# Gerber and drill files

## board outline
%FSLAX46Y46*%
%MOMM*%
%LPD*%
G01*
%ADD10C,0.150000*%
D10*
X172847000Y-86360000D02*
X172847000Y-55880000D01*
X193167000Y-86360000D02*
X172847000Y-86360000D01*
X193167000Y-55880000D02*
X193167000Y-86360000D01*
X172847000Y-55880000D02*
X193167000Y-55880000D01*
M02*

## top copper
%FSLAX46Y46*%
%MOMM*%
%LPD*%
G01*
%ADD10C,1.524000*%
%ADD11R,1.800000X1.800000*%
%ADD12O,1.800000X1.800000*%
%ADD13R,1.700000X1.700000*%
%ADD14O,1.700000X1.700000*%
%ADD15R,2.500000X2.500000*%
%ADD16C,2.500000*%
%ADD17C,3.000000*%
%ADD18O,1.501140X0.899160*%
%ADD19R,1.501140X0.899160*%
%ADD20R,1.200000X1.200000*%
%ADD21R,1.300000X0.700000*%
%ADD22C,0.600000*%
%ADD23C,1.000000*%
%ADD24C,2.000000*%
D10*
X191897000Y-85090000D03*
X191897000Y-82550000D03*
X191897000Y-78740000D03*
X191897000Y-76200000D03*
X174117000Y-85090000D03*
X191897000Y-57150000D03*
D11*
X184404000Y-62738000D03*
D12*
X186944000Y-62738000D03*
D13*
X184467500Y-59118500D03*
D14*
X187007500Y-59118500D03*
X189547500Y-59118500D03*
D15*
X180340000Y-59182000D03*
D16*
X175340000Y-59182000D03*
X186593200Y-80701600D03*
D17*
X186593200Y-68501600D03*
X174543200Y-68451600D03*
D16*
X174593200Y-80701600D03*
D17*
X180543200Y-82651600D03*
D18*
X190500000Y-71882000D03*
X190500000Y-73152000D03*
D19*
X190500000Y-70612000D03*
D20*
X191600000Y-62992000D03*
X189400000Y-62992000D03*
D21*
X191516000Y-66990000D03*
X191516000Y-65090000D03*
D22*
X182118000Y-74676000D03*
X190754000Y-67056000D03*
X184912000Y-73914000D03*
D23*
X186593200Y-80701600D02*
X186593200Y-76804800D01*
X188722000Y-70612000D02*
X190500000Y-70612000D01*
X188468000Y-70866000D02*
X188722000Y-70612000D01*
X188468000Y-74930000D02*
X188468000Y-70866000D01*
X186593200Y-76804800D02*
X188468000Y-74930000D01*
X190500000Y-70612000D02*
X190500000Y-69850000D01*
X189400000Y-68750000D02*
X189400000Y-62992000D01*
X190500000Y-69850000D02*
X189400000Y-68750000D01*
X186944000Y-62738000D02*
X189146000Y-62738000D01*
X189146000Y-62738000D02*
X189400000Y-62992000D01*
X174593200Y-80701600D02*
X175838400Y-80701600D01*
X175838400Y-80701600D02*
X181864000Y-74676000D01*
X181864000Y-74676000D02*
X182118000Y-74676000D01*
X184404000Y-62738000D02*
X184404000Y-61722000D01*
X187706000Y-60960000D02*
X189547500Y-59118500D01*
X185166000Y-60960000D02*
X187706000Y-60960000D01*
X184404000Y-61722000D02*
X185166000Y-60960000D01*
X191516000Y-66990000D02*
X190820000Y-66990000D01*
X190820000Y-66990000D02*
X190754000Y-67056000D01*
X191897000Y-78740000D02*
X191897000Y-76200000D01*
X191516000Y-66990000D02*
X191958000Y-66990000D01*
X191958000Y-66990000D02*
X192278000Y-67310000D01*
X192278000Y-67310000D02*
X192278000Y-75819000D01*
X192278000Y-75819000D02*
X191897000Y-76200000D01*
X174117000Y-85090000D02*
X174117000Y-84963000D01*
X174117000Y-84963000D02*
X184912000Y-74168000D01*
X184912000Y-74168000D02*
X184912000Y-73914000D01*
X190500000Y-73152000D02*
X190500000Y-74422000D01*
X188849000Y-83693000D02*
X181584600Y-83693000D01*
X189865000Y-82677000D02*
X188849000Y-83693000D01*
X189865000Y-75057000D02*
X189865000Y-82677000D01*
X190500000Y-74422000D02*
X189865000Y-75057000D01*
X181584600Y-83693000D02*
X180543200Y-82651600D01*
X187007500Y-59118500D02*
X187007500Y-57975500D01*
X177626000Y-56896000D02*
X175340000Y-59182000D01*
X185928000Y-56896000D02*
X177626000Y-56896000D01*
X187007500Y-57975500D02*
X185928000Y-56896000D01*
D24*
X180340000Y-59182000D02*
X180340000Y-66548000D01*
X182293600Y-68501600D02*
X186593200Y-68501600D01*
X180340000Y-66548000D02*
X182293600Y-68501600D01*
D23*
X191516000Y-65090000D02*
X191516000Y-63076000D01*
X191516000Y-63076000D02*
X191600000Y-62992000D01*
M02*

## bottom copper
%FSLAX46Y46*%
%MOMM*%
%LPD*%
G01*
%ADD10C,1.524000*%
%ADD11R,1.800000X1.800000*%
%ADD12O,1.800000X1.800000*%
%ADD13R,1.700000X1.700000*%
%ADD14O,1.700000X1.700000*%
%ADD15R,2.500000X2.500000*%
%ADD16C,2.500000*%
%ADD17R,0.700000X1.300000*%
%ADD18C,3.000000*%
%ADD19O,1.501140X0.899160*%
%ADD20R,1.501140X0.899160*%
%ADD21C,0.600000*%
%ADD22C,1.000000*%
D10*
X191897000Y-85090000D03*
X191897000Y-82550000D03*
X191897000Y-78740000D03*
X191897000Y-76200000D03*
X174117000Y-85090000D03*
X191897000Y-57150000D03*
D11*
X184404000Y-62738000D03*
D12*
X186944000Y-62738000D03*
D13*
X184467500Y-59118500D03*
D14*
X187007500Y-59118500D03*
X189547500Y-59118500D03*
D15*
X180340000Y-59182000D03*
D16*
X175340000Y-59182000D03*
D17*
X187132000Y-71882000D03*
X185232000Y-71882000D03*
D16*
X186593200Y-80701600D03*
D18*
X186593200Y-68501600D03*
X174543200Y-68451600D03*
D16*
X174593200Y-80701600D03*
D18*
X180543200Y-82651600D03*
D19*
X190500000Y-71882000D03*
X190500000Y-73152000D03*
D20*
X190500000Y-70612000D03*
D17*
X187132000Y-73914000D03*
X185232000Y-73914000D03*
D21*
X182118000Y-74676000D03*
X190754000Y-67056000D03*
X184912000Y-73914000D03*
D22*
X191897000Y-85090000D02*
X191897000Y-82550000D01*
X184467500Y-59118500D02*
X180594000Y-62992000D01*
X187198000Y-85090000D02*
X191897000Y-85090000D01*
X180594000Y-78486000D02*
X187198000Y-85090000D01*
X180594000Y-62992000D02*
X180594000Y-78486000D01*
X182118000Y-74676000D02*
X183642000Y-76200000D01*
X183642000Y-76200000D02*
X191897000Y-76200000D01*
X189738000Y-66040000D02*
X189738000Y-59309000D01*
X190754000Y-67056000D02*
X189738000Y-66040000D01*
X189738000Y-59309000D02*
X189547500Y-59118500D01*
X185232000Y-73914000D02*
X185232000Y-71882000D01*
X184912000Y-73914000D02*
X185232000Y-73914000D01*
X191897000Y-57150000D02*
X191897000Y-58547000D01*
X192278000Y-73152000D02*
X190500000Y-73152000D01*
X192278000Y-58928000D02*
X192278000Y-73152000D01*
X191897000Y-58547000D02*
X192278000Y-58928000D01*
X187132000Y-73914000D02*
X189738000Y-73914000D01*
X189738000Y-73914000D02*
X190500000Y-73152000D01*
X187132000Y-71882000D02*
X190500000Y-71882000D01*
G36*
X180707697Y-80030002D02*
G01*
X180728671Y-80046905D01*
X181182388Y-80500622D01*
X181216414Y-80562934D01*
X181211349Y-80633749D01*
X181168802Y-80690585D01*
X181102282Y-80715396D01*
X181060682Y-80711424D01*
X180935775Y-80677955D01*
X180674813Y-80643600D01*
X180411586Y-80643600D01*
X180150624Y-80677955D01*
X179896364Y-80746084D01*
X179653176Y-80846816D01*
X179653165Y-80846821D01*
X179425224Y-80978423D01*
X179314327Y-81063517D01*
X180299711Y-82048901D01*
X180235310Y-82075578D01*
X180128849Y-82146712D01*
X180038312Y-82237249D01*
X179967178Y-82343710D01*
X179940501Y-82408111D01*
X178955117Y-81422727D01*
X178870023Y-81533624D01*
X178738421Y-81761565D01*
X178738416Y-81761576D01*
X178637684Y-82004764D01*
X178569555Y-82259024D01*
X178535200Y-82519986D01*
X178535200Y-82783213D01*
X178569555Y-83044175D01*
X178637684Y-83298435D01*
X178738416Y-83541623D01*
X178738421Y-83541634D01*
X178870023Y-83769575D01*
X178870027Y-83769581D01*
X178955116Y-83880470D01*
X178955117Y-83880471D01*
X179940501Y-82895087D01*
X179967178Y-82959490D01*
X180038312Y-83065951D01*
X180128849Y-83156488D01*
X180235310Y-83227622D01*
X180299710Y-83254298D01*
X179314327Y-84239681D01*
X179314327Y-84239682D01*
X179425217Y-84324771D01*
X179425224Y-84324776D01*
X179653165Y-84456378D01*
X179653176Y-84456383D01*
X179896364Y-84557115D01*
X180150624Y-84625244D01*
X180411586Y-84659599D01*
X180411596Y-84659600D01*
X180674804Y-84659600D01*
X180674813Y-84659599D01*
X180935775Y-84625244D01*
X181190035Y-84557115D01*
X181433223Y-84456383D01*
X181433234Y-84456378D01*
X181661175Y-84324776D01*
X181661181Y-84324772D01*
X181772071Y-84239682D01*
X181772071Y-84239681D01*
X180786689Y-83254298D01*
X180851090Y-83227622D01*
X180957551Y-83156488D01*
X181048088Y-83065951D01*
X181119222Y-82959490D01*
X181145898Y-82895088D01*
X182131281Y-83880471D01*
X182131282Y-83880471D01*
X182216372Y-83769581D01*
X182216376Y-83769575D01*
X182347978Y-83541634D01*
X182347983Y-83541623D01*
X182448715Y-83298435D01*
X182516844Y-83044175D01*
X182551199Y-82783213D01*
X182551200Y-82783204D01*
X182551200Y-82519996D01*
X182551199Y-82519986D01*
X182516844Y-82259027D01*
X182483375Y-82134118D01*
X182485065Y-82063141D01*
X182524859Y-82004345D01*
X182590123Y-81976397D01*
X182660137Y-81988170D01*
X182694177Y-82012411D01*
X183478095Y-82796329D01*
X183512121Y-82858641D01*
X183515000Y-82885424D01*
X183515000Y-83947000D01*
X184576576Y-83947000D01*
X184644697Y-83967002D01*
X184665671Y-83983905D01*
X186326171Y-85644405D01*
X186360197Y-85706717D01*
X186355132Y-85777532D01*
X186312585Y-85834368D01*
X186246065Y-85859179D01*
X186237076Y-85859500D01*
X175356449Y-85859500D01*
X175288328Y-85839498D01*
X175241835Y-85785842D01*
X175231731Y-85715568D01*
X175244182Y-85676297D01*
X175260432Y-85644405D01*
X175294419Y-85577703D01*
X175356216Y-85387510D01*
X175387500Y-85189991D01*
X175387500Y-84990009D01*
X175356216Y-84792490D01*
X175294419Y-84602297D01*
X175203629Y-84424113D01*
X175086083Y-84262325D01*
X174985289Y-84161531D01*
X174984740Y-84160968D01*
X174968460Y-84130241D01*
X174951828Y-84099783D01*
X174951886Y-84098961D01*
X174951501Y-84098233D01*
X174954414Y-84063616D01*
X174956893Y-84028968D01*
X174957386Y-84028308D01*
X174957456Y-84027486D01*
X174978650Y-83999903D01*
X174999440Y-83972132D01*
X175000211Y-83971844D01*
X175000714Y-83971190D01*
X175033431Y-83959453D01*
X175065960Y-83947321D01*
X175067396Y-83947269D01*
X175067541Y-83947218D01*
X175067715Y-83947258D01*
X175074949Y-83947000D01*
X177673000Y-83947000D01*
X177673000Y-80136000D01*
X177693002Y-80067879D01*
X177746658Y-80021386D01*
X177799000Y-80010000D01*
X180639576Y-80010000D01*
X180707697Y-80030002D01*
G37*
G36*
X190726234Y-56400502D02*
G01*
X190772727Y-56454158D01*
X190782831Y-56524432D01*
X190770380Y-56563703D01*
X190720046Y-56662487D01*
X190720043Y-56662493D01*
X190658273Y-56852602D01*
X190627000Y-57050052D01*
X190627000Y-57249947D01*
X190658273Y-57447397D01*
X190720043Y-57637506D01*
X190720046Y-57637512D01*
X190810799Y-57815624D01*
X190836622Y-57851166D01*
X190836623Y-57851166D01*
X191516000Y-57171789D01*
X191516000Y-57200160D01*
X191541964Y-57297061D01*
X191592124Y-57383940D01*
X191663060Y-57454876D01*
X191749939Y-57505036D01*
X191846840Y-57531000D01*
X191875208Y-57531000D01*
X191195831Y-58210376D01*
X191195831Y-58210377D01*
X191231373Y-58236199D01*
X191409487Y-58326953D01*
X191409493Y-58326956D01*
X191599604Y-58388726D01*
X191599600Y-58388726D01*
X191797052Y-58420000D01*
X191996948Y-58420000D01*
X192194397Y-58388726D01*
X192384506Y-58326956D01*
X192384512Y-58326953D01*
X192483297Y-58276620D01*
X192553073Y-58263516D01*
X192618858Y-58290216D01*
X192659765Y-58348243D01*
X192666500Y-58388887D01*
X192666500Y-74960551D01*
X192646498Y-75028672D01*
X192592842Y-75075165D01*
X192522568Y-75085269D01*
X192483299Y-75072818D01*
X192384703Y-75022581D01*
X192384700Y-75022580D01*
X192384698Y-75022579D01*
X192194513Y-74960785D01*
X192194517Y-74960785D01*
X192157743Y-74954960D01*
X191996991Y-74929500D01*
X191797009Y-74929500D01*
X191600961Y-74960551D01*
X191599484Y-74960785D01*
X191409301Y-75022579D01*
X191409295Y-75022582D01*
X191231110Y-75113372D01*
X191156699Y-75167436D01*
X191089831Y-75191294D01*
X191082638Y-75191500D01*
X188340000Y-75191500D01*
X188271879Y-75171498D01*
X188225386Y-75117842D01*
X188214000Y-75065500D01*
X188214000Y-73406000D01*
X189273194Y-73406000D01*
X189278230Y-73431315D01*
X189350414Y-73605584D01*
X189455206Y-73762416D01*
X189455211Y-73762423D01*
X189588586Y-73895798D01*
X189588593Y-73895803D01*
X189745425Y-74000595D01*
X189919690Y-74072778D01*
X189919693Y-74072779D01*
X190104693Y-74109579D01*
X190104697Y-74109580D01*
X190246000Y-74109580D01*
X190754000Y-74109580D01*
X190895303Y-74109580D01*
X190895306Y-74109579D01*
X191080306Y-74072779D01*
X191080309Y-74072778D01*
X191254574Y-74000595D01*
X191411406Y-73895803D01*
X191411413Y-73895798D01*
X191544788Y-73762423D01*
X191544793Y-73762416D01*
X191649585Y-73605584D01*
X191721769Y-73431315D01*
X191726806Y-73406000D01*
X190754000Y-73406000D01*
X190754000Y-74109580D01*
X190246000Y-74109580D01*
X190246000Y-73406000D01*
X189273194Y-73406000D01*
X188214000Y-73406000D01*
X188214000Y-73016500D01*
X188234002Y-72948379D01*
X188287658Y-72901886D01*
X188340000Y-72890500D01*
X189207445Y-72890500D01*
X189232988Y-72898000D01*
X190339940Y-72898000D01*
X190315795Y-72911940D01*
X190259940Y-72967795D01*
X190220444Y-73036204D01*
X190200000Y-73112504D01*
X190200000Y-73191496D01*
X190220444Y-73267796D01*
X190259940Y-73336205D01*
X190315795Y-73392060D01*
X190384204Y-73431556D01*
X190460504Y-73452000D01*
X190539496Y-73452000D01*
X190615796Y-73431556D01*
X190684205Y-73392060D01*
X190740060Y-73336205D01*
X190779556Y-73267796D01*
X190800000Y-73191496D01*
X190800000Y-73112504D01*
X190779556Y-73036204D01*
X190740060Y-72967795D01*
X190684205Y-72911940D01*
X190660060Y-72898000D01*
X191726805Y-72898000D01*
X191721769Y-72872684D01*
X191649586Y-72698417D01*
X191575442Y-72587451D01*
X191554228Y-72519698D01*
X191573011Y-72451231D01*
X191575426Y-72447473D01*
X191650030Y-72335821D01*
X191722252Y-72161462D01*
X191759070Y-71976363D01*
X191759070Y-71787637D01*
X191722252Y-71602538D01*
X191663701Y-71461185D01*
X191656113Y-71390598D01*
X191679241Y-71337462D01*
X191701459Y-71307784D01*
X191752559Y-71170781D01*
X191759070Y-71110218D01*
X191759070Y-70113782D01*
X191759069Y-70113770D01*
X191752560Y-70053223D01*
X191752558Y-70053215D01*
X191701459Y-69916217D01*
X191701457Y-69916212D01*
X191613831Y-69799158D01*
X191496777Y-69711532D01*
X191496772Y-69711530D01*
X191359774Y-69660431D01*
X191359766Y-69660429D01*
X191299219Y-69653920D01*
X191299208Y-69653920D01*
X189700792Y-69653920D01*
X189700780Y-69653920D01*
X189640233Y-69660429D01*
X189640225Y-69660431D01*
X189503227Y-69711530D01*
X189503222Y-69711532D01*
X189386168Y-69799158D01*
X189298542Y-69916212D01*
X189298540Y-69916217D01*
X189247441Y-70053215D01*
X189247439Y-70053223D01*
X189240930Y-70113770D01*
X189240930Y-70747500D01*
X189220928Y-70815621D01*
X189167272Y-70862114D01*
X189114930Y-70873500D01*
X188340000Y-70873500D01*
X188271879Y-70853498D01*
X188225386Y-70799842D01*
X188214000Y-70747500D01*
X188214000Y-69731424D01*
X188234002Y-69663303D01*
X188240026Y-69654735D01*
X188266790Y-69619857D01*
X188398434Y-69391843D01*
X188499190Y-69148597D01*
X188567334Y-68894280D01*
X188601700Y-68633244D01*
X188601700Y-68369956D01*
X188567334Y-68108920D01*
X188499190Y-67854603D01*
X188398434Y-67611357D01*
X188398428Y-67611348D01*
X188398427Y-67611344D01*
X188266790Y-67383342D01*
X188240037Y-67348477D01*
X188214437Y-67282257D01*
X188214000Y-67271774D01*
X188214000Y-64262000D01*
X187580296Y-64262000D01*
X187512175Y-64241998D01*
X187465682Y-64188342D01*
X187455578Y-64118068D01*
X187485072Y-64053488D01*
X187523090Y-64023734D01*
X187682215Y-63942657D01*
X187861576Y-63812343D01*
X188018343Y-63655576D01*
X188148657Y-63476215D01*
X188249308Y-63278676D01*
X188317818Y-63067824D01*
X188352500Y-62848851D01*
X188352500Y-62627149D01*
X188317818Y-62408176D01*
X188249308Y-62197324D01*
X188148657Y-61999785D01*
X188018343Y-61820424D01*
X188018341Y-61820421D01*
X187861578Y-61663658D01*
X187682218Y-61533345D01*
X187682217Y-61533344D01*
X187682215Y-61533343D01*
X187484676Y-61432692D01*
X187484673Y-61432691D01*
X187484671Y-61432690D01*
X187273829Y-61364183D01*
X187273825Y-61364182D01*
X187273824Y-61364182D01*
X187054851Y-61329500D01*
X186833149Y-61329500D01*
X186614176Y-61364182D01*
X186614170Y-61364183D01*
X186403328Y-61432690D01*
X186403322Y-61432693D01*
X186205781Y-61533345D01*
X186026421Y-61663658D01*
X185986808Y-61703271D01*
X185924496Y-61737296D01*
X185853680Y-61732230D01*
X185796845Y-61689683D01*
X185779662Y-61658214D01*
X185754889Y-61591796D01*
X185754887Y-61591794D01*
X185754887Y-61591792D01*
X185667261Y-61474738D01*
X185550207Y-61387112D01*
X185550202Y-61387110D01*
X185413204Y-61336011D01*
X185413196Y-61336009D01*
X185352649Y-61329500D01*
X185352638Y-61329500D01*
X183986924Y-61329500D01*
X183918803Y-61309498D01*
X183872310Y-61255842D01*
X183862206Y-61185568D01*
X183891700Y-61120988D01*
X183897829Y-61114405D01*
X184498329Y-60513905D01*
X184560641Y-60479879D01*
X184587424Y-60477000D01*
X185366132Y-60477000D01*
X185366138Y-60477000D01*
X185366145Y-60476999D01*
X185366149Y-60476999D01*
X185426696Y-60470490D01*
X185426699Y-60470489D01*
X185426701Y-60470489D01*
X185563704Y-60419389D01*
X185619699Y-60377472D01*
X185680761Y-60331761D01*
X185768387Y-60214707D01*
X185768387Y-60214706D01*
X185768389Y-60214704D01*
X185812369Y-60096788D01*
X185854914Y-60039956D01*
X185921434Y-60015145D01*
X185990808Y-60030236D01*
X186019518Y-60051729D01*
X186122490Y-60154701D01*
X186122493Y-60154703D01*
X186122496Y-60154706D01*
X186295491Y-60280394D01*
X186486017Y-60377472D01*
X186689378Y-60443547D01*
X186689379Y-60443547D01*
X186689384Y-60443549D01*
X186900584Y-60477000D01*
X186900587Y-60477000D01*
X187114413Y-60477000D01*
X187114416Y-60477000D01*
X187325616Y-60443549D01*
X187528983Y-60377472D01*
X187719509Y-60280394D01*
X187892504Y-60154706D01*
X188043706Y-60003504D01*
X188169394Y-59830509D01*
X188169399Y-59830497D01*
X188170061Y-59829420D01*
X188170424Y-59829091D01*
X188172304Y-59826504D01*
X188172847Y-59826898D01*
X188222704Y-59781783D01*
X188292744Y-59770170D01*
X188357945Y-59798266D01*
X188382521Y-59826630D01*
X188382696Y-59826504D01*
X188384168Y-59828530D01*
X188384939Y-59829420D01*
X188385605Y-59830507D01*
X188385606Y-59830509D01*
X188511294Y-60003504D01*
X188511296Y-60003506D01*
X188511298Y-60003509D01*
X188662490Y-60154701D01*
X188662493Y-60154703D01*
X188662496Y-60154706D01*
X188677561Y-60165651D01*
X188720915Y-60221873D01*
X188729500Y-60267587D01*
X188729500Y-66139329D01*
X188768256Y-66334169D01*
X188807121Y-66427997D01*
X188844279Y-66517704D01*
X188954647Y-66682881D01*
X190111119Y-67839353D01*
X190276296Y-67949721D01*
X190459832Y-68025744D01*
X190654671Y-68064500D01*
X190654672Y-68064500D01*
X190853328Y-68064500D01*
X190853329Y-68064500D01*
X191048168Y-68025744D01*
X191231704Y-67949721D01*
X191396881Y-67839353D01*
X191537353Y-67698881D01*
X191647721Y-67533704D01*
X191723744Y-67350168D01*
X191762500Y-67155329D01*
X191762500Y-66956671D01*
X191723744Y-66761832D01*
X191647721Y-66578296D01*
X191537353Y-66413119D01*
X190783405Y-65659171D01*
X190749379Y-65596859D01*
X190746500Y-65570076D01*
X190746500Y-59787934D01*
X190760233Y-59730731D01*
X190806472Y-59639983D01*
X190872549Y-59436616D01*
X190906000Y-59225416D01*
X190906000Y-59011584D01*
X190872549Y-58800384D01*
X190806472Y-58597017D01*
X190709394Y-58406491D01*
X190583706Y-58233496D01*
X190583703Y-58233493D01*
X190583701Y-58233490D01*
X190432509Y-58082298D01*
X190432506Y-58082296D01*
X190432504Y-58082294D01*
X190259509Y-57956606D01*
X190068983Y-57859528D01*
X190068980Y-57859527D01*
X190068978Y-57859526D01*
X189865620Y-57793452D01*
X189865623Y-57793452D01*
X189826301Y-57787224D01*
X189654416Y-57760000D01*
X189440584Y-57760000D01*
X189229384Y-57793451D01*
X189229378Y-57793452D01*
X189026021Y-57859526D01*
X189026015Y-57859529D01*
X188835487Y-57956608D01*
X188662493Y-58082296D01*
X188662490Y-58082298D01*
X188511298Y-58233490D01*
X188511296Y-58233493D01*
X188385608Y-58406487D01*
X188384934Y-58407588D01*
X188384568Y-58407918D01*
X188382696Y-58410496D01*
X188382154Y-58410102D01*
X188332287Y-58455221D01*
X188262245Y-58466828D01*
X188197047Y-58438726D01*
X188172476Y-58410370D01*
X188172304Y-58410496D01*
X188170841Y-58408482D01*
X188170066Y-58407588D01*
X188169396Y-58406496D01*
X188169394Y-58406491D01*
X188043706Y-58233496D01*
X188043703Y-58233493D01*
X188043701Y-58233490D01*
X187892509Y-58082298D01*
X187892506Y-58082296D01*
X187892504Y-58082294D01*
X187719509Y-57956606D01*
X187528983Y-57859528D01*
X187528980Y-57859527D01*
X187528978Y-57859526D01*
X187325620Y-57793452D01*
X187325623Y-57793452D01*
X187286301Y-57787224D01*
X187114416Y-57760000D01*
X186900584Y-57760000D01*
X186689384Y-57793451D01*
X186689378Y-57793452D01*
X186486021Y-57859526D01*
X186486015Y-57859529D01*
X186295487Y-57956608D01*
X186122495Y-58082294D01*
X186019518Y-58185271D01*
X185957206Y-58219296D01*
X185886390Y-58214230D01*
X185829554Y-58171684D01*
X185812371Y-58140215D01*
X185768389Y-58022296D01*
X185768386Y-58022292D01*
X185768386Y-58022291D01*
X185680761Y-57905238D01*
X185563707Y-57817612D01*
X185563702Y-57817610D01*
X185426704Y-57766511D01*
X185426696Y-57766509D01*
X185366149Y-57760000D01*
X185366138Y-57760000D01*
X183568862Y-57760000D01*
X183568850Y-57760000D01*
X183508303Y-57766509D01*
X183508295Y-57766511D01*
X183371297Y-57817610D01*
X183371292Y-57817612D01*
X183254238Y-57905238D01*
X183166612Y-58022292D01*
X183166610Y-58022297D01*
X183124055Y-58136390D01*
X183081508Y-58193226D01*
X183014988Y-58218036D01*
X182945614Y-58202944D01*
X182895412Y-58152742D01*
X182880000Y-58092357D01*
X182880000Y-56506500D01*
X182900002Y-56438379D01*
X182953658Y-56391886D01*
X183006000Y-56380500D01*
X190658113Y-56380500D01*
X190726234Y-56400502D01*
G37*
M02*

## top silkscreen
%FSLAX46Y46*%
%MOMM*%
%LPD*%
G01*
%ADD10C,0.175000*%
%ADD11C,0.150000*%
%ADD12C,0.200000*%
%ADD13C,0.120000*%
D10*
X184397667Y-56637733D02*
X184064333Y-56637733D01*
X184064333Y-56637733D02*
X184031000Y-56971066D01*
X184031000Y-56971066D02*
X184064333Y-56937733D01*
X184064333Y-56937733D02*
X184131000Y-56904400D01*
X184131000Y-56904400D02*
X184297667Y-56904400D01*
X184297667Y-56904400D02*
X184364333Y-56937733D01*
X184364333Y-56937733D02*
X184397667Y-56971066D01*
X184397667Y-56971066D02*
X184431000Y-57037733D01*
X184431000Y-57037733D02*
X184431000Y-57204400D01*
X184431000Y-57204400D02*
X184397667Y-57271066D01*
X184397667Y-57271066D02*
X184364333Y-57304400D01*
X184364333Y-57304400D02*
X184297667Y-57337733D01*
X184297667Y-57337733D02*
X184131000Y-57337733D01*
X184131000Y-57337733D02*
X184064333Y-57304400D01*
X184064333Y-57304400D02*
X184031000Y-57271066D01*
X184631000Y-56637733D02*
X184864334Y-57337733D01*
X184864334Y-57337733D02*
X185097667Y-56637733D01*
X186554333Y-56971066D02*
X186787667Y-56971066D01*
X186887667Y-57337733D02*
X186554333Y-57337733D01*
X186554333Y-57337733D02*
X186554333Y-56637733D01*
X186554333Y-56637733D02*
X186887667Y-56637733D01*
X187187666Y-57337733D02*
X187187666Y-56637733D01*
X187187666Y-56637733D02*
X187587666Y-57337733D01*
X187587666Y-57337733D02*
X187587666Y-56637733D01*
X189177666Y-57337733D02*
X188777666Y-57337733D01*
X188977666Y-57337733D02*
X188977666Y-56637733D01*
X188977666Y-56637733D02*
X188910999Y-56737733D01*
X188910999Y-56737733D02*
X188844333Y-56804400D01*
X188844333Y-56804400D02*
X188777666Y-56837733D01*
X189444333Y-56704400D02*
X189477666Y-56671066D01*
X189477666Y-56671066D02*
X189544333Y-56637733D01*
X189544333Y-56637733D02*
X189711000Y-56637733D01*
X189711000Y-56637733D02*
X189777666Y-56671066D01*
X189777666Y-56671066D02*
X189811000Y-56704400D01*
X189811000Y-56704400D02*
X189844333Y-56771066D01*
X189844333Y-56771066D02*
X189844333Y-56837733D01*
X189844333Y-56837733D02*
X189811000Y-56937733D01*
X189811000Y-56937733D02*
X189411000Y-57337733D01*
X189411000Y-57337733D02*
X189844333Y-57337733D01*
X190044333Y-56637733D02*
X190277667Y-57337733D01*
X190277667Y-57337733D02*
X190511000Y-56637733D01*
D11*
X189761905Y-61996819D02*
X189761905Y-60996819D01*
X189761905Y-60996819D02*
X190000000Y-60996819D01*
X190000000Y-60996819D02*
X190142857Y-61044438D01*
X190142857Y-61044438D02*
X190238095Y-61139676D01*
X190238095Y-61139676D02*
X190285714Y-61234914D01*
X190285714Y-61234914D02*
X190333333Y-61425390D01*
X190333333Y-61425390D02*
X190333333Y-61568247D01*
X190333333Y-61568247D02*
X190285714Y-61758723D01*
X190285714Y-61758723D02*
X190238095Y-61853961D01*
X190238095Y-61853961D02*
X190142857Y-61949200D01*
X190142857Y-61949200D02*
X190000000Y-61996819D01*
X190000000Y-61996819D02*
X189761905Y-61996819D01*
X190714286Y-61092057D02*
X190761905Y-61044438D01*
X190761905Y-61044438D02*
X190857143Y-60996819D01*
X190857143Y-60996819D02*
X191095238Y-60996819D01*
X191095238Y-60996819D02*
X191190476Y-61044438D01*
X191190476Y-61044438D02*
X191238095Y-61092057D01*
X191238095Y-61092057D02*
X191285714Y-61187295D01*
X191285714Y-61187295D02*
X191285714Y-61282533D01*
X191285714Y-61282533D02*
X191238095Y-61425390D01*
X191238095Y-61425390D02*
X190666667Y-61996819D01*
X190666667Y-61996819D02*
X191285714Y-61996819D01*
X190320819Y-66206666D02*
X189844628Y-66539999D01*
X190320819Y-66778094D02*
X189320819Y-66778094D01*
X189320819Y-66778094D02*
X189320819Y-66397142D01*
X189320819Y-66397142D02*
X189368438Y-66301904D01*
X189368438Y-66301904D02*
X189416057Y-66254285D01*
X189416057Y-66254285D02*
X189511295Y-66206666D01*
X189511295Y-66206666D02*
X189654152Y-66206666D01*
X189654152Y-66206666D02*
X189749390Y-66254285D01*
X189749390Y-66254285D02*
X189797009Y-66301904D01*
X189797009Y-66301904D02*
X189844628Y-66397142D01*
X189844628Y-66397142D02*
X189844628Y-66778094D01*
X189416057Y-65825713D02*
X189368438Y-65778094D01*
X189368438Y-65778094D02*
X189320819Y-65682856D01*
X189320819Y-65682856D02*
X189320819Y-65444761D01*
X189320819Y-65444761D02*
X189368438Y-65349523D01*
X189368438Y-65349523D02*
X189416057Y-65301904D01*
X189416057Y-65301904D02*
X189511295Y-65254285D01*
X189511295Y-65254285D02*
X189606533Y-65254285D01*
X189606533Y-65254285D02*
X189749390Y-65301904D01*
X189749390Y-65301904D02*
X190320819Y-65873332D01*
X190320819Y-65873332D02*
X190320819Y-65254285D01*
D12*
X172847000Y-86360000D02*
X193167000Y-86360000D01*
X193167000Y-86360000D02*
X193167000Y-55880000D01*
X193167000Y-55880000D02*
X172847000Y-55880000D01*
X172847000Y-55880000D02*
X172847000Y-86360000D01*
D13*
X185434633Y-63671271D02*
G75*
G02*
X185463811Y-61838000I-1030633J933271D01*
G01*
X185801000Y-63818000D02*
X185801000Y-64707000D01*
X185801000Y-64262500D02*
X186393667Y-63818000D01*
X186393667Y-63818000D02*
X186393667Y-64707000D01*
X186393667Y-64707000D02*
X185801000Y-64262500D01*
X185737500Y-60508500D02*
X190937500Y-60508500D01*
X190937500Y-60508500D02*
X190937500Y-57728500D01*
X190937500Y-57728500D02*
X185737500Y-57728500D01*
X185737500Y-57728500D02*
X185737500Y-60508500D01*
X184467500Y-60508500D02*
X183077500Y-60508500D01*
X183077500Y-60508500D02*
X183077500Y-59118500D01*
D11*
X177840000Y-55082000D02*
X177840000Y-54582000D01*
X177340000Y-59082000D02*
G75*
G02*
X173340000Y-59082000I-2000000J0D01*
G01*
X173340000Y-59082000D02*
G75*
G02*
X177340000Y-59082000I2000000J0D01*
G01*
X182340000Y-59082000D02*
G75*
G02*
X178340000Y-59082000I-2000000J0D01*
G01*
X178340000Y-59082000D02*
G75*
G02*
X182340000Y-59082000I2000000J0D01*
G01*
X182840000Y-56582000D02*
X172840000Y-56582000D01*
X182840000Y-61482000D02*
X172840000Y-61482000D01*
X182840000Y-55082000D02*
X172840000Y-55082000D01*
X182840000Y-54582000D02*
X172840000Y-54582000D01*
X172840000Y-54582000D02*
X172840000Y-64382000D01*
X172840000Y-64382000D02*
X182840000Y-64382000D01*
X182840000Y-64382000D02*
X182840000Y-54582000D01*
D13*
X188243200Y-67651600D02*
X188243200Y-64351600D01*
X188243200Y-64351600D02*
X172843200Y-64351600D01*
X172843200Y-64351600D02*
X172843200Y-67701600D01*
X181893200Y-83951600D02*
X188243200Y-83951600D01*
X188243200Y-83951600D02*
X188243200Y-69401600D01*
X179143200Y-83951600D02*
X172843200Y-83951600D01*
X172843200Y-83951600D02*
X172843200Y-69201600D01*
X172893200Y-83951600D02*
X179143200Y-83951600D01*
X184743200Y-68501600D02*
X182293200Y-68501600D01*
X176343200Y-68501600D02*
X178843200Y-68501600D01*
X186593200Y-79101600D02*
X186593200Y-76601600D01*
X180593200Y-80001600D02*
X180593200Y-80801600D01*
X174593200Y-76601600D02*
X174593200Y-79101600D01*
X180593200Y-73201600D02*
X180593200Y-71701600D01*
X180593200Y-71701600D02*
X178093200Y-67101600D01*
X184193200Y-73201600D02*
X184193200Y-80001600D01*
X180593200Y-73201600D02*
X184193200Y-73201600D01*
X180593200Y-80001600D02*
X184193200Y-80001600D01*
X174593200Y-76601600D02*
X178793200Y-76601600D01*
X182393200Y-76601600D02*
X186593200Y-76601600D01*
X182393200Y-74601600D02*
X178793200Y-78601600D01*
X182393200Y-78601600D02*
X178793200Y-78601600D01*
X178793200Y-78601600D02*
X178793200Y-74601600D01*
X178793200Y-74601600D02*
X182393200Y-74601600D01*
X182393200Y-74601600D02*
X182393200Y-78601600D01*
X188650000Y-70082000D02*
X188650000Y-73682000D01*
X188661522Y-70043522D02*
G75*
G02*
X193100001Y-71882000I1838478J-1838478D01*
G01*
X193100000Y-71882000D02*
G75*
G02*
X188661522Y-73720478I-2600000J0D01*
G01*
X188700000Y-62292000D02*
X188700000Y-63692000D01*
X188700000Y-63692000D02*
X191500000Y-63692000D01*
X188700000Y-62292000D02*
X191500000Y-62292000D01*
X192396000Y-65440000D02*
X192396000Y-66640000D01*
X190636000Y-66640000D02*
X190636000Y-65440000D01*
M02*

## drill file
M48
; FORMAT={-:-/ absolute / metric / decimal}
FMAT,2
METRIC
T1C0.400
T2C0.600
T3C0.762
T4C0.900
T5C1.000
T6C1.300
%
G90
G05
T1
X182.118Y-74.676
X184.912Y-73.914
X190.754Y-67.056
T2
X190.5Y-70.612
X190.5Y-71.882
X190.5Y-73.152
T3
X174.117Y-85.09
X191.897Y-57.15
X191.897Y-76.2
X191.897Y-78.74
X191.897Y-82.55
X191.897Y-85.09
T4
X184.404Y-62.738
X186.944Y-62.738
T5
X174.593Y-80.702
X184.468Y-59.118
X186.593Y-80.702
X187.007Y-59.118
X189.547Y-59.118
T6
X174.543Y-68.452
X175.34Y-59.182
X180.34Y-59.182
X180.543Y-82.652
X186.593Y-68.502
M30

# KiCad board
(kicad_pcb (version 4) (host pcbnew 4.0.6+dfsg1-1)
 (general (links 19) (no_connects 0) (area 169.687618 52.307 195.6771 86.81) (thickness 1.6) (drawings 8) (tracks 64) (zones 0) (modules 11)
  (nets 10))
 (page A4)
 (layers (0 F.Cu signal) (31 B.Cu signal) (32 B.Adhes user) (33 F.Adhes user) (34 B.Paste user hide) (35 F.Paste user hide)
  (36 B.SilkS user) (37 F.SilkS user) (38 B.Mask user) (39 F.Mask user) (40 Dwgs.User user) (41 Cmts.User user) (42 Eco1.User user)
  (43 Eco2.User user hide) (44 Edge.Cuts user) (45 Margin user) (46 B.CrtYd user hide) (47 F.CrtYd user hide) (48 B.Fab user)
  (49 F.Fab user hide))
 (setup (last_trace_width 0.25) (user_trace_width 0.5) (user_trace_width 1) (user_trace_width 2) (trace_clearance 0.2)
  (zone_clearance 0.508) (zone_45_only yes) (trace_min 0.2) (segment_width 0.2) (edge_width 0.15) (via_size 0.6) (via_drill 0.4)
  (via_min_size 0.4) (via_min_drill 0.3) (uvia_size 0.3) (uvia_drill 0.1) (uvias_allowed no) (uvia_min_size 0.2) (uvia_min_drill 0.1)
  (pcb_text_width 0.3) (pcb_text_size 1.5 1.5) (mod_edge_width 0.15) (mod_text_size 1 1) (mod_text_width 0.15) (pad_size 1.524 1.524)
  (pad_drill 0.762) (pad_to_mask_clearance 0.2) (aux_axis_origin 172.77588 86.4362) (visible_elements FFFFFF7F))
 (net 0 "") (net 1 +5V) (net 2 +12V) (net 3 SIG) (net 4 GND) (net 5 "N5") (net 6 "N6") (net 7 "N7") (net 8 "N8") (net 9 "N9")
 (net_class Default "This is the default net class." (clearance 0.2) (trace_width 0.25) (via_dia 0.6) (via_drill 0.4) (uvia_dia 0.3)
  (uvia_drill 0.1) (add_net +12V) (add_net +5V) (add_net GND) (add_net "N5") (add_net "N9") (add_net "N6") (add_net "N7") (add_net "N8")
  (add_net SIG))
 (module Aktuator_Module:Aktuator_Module (layer F.Cu) (at 172.847 86.36)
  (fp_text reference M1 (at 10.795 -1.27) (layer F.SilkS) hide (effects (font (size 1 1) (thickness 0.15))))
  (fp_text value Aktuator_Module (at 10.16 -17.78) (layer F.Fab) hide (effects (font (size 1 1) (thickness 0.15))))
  (fp_line (start 0 0) (end 20.32 0) (layer F.SilkS) (width 0.2))
  (fp_line (start 20.32 0) (end 20.32 -30.48) (layer F.SilkS) (width 0.2))
  (fp_line (start 20.32 -30.48) (end 0 -30.48) (layer F.SilkS) (width 0.2))
  (fp_line (start 0 -30.48) (end 0 0) (layer F.SilkS) (width 0.2))
  (pad 1 thru_hole circle (at 19.05 -1.27) (size 1.524 1.524) (drill 0.762) (layers *.Cu *.Mask) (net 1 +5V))
  (pad 1 thru_hole circle (at 19.05 -3.81) (size 1.524 1.524) (drill 0.762) (layers *.Cu *.Mask) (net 1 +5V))
  (pad 2 thru_hole circle (at 19.05 -7.62) (size 1.524 1.524) (drill 0.762) (layers *.Cu *.Mask) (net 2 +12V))
  (pad 2 thru_hole circle (at 19.05 -10.16) (size 1.524 1.524) (drill 0.762) (layers *.Cu *.Mask) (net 2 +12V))
  (pad 3 thru_hole circle (at 1.27 -1.27) (size 1.524 1.524) (drill 0.762) (layers *.Cu *.Mask) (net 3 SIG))
  (pad 4 thru_hole circle (at 19.05 -29.21) (size 1.524 1.524) (drill 0.762) (layers *.Cu *.Mask) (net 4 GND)))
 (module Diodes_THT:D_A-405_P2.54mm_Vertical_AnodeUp (layer F.Cu) (at 184.404 62.738)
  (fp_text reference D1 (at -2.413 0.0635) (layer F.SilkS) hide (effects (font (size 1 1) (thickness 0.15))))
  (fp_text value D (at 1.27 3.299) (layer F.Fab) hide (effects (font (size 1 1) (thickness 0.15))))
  (fp_arc (start 0 0) (end 1.059811 -0.9) (angle -277.5) (layer F.SilkS) (width 0.12))
  (fp_line (start 1.397 1.08) (end 1.397 1.969) (layer F.SilkS) (width 0.12))
  (fp_line (start 1.397 1.5245) (end 1.989667 1.08) (layer F.SilkS) (width 0.12))
  (fp_line (start 1.989667 1.08) (end 1.989667 1.969) (layer F.SilkS) (width 0.12))
  (fp_line (start 1.989667 1.969) (end 1.397 1.5245) (layer F.SilkS) (width 0.12))
  (pad 1 thru_hole rect (at 0 0) (size 1.8 1.8) (drill 0.9) (layers *.Cu *.Mask) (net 2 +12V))
  (pad 2 thru_hole oval (at 2.54 0) (size 1.8 1.8) (drill 0.9) (layers *.Cu *.Mask) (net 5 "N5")))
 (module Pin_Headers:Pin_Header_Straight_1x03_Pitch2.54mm (layer F.Cu) (at 184.4675 59.1185 90)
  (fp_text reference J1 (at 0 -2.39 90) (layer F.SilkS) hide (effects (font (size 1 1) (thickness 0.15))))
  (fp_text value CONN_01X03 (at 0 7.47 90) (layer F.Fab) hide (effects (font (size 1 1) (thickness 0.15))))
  (fp_line (start -1.39 1.27) (end -1.39 6.47) (layer F.SilkS) (width 0.12))
  (fp_line (start -1.39 6.47) (end 1.39 6.47) (layer F.SilkS) (width 0.12))
  (fp_line (start 1.39 6.47) (end 1.39 1.27) (layer F.SilkS) (width 0.12))
  (fp_line (start 1.39 1.27) (end -1.39 1.27) (layer F.SilkS) (width 0.12))
  (fp_line (start -1.39 0) (end -1.39 -1.39) (layer F.SilkS) (width 0.12))
  (fp_line (start -1.39 -1.39) (end 0 -1.39) (layer F.SilkS) (width 0.12))
  (pad 1 thru_hole rect (at 0 0 90) (size 1.7 1.7) (drill 1) (layers *.Cu *.Mask) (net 1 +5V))
  (pad 2 thru_hole oval (at 0 2.54 90) (size 1.7 1.7) (drill 1) (layers *.Cu *.Mask) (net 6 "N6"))
  (pad 3 thru_hole oval (at 0 5.08 90) (size 1.7 1.7) (drill 1) (layers *.Cu *.Mask) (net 2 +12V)))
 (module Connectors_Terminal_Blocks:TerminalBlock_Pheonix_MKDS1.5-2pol (layer F.Cu) (at 180.34 59.182 180)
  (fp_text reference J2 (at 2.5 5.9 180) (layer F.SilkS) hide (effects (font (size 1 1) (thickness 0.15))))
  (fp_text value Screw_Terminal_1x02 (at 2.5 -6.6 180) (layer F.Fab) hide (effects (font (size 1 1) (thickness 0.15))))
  (fp_line (start 2.5 4.1) (end 2.5 4.6) (layer F.SilkS) (width 0.15))
  (fp_circle (center 5 0.1) (end 3 0.1) (layer F.SilkS) (width 0.15))
  (fp_circle (center 0 0.1) (end 2 0.1) (layer F.SilkS) (width 0.15))
  (fp_line (start -2.5 2.6) (end 7.5 2.6) (layer F.SilkS) (width 0.15))
  (fp_line (start -2.5 -2.3) (end 7.5 -2.3) (layer F.SilkS) (width 0.15))
  (fp_line (start -2.5 4.1) (end 7.5 4.1) (layer F.SilkS) (width 0.15))
  (fp_line (start -2.5 4.6) (end 7.5 4.6) (layer F.SilkS) (width 0.15))
  (fp_line (start 7.5 4.6) (end 7.5 -5.2) (layer F.SilkS) (width 0.15))
  (fp_line (start 7.5 -5.2) (end -2.5 -5.2) (layer F.SilkS) (width 0.15))
  (fp_line (start -2.5 -5.2) (end -2.5 4.6) (layer F.SilkS) (width 0.15))
  (pad 1 thru_hole rect (at 0 0 180) (size 2.5 2.5) (drill 1.3) (layers *.Cu *.Mask) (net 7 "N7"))
  (pad 2 thru_hole circle (at 5 0 180) (size 2.5 2.5) (drill 1.3) (layers *.Cu *.Mask) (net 6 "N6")))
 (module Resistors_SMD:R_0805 (layer B.Cu) (at 186.182 71.882 180)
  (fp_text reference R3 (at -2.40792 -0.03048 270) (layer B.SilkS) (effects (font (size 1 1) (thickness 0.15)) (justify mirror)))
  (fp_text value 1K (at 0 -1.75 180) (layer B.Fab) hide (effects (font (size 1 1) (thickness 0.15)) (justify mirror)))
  (pad 1 smd rect (at -0.95 0 180) (size 0.7 1.3) (layers B.Cu B.Paste B.Mask) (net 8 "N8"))
  (pad 2 smd rect (at 0.95 0 180) (size 0.7 1.3) (layers B.Cu B.Paste B.Mask) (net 3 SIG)))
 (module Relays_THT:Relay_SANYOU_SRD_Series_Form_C (layer F.Cu) (at 180.5432 82.6516 90)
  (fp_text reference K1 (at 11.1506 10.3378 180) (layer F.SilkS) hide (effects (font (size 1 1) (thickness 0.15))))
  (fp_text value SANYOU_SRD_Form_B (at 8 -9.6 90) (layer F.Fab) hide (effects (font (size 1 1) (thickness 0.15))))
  (fp_line (start 15 7.7) (end 18.3 7.7) (layer F.SilkS) (width 0.12))
  (fp_line (start 18.3 7.7) (end 18.3 -7.7) (layer F.SilkS) (width 0.12))
  (fp_line (start 18.3 -7.7) (end 14.95 -7.7) (layer F.SilkS) (width 0.12))
  (fp_line (start -1.3 1.35) (end -1.3 7.7) (layer F.SilkS) (width 0.12))
  (fp_line (start -1.3 7.7) (end 13.25 7.7) (layer F.SilkS) (width 0.12))
  (fp_line (start -1.3 -1.4) (end -1.3 -7.7) (layer F.SilkS) (width 0.12))
  (fp_line (start -1.3 -7.7) (end 13.45 -7.7) (layer F.SilkS) (width 0.12))
  (fp_line (start -1.3 -7.65) (end -1.3 -1.4) (layer F.SilkS) (width 0.12))
  (fp_line (start 14.15 4.2) (end 14.15 1.75) (layer F.SilkS) (width 0.12))
  (fp_line (start 14.15 -4.2) (end 14.15 -1.7) (layer F.SilkS) (width 0.12))
  (fp_line (start 3.55 6.05) (end 6.05 6.05) (layer F.SilkS) (width 0.12))
  (fp_line (start 2.65 0.05) (end 1.85 0.05) (layer F.SilkS) (width 0.12))
  (fp_line (start 6.05 -5.95) (end 3.55 -5.95) (layer F.SilkS) (width 0.12))
  (fp_line (start 9.45 0.05) (end 10.95 0.05) (layer F.SilkS) (width 0.12))
  (fp_line (start 10.95 0.05) (end 15.55 -2.45) (layer F.SilkS) (width 0.12))
  (fp_line (start 9.45 3.65) (end 2.65 3.65) (layer F.SilkS) (width 0.12))
  (fp_line (start 9.45 0.05) (end 9.45 3.65) (layer F.SilkS) (width 0.12))
  (fp_line (start 2.65 0.05) (end 2.65 3.65) (layer F.SilkS) (width 0.12))
  (fp_line (start 6.05 -5.95) (end 6.05 -1.75) (layer F.SilkS) (width 0.12))
  (fp_line (start 6.05 1.85) (end 6.05 6.05) (layer F.SilkS) (width 0.12))
  (fp_line (start 8.05 1.85) (end 4.05 -1.75) (layer F.SilkS) (width 0.12))
  (fp_line (start 4.05 1.85) (end 4.05 -1.75) (layer F.SilkS) (width 0.12))
  (fp_line (start 4.05 -1.75) (end 8.05 -1.75) (layer F.SilkS) (width 0.12))
  (fp_line (start 8.05 -1.75) (end 8.05 1.85) (layer F.SilkS) (width 0.12))
  (fp_line (start 8.05 1.85) (end 4.05 1.85) (layer F.SilkS) (width 0.12))
  (pad 2 thru_hole circle (at 1.95 6.05 180) (size 2.5 2.5) (drill 1) (layers *.Cu *.Mask) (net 5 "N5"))
  (pad 3 thru_hole circle (at 14.15 6.05 180) (size 3 3) (drill 1.3) (layers *.Cu *.Mask) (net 7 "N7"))
  (pad 4 thru_hole circle (at 14.2 -6 180) (size 3 3) (drill 1.3) (layers *.Cu *.Mask))
  (pad 5 thru_hole circle (at 1.95 -5.95 180) (size 2.5 2.5) (drill 1) (layers *.Cu *.Mask) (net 2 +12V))
  (pad 1 thru_hole circle (at 0 0 180) (size 3 3) (drill 1.3) (layers *.Cu *.Mask) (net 4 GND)))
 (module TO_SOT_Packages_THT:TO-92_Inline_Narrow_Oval (layer F.Cu) (at 190.5 70.612 270)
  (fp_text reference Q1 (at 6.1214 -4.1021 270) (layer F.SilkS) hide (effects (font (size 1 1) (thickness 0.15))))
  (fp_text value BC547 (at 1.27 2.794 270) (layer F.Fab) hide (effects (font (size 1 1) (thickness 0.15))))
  (fp_line (start -0.53 1.85) (end 3.07 1.85) (layer F.SilkS) (width 0.12))
  (fp_arc (start 1.27 0) (end 1.27 -2.6) (angle -135) (layer F.SilkS) (width 0.12))
  (fp_arc (start 1.27 0) (end 1.27 -2.6) (angle 135) (layer F.SilkS) (width 0.12))
  (pad 2 thru_hole oval (at 1.27 0 90) (size 0.89916 1.50114) (drill 0.6) (layers *.Cu *.Mask) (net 8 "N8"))
  (pad 3 thru_hole oval (at 2.54 0 90) (size 0.89916 1.50114) (drill 0.6) (layers *.Cu *.Mask) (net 4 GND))
  (pad 1 thru_hole rect (at 0 0 90) (size 0.89916 1.50114) (drill 0.6) (layers *.Cu *.Mask) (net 5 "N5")))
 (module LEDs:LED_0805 (layer F.Cu) (at 190.5 62.992)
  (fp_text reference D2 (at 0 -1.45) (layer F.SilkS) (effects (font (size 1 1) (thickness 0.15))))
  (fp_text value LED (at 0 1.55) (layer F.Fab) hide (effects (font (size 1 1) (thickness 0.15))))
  (fp_line (start -1.8 -0.7) (end -1.8 0.7) (layer F.SilkS) (width 0.12))
  (fp_line (start -1.8 0.7) (end 1 0.7) (layer F.SilkS) (width 0.12))
  (fp_line (start -1.8 -0.7) (end 1 -0.7) (layer F.SilkS) (width 0.12))
  (pad 2 smd rect (at 1.1 0 180) (size 1.2 1.2) (layers F.Cu F.Paste F.Mask) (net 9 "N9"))
  (pad 1 smd rect (at -1.1 0 180) (size 1.2 1.2) (layers F.Cu F.Paste F.Mask) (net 5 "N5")))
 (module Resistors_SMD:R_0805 (layer B.Cu) (at 186.182 73.914 180)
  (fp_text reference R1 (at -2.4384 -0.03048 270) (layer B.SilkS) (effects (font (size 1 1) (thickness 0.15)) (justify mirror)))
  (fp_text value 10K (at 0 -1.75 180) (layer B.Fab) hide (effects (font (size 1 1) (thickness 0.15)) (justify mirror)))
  (pad 1 smd rect (at -0.95 0 180) (size 0.7 1.3) (layers B.Cu B.Paste B.Mask) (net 4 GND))
  (pad 2 smd rect (at 0.95 0 180) (size 0.7 1.3) (layers B.Cu B.Paste B.Mask) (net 3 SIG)))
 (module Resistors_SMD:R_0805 (layer F.Cu) (at 191.516 66.04 90)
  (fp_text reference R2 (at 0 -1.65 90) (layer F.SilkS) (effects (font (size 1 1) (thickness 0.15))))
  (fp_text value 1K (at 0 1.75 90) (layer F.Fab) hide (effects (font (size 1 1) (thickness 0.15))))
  (fp_line (start 0.6 0.88) (end -0.6 0.88) (layer F.SilkS) (width 0.12))
  (fp_line (start -0.6 -0.88) (end 0.6 -0.88) (layer F.SilkS) (width 0.12))
  (pad 1 smd rect (at -0.95 0 90) (size 0.7 1.3) (layers F.Cu F.Paste F.Mask) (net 2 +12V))
  (pad 2 smd rect (at 0.95 0 90) (size 0.7 1.3) (layers F.Cu F.Paste F.Mask) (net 9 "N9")))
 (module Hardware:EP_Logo (layer B.Cu) (at 179.451 74.676 180)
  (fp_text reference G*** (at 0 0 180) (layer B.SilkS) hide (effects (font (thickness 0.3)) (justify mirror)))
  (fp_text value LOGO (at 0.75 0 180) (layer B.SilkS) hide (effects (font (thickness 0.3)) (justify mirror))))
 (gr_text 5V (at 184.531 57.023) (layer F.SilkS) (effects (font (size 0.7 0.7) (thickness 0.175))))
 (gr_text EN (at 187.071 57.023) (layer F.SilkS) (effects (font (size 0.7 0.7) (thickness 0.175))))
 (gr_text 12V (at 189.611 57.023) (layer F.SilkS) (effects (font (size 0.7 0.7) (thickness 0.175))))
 (gr_line (start 172.847 86.36) (end 172.847 55.88) (angle 90) (layer Edge.Cuts) (width 0.15))
 (gr_line (start 193.167 86.36) (end 172.847 86.36) (angle 90) (layer Edge.Cuts) (width 0.15))
 (gr_line (start 193.167 55.88) (end 193.167 86.36) (angle 90) (layer Edge.Cuts) (width 0.15))
 (gr_line (start 172.847 55.88) (end 193.167 55.88) (angle 90) (layer Edge.Cuts) (width 0.15))
 (segment (start 186.5932 80.7016) (end 186.5932 76.8048) (width 1) (layer F.Cu) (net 5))
 (segment (start 188.722 70.612) (end 190.5 70.612) (width 1) (layer F.Cu) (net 5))
 (segment (start 188.468 70.866) (end 188.722 70.612) (width 1) (layer F.Cu) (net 5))
 (segment (start 188.468 74.93) (end 188.468 70.866) (width 1) (layer F.Cu) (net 5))
 (segment (start 186.5932 76.8048) (end 188.468 74.93) (width 1) (layer F.Cu) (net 5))
 (segment (start 190.5 70.612) (end 190.5 69.85) (width 1) (layer F.Cu) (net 5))
 (segment (start 189.4 68.75) (end 189.4 62.992) (width 1) (layer F.Cu) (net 5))
 (segment (start 190.5 69.85) (end 189.4 68.75) (width 1) (layer F.Cu) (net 5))
 (segment (start 186.944 62.738) (end 189.146 62.738) (width 1) (layer F.Cu) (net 5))
 (segment (start 189.146 62.738) (end 189.4 62.992) (width 1) (layer F.Cu) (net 5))
 (segment (start 191.897 85.09) (end 191.897 82.55) (width 1) (layer B.Cu) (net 1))
 (segment (start 184.4675 59.1185) (end 180.594 62.992) (width 1) (layer B.Cu) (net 1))
 (segment (start 187.198 85.09) (end 191.897 85.09) (width 1) (layer B.Cu) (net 1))
 (segment (start 180.594 78.486) (end 187.198 85.09) (width 1) (layer B.Cu) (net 1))
 (segment (start 180.594 62.992) (end 180.594 78.486) (width 1) (layer B.Cu) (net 1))
 (segment (start 174.5932 80.7016) (end 175.8384 80.7016) (width 1) (layer F.Cu) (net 2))
 (segment (start 175.8384 80.7016) (end 181.864 74.676) (width 1) (layer F.Cu) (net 2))
 (segment (start 181.864 74.676) (end 182.118 74.676) (width 1) (layer F.Cu) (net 2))
 (via (at 182.118 74.676) (size 0.6) (drill 0.4) (layers F.Cu B.Cu) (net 2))
 (segment (start 182.118 74.676) (end 183.642 76.2) (width 1) (layer B.Cu) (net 2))
 (segment (start 183.642 76.2) (end 191.897 76.2) (width 1) (layer B.Cu) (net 2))
 (segment (start 184.404 62.738) (end 184.404 61.722) (width 1) (layer F.Cu) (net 2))
 (segment (start 187.706 60.96) (end 189.5475 59.1185) (width 1) (layer F.Cu) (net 2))
 (segment (start 185.166 60.96) (end 187.706 60.96) (width 1) (layer F.Cu) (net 2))
 (segment (start 184.404 61.722) (end 185.166 60.96) (width 1) (layer F.Cu) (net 2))
 (segment (start 191.516 66.99) (end 190.82 66.99) (width 1) (layer F.Cu) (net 2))
 (segment (start 189.738 66.04) (end 189.738 59.309) (width 1) (layer B.Cu) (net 2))
 (segment (start 190.754 67.056) (end 189.738 66.04) (width 1) (layer B.Cu) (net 2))
 (via (at 190.754 67.056) (size 0.6) (drill 0.4) (layers F.Cu B.Cu) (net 2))
 (segment (start 190.82 66.99) (end 190.754 67.056) (width 1) (layer F.Cu) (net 2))
 (segment (start 189.738 59.309) (end 189.5475 59.1185) (width 1) (layer B.Cu) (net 2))
 (segment (start 191.897 78.74) (end 191.897 76.2) (width 1) (layer F.Cu) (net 2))
 (segment (start 191.516 66.99) (end 191.958 66.99) (width 1) (layer F.Cu) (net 2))
 (segment (start 191.958 66.99) (end 192.278 67.31) (width 1) (layer F.Cu) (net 2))
 (segment (start 192.278 67.31) (end 192.278 75.819) (width 1) (layer F.Cu) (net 2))
 (segment (start 192.278 75.819) (end 191.897 76.2) (width 1) (layer F.Cu) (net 2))
 (segment (start 185.232 73.914) (end 185.232 71.882) (width 1) (layer B.Cu) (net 3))
 (segment (start 174.117 85.09) (end 174.117 84.963) (width 1) (layer F.Cu) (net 3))
 (segment (start 174.117 84.963) (end 184.912 74.168) (width 1) (layer F.Cu) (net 3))
 (segment (start 184.912 74.168) (end 184.912 73.914) (width 1) (layer F.Cu) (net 3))
 (via (at 184.912 73.914) (size 0.6) (drill 0.4) (layers F.Cu B.Cu) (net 3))
 (segment (start 184.912 73.914) (end 185.232 73.914) (width 1) (layer B.Cu) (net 3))
 (segment (start 190.5 73.152) (end 190.5 74.422) (width 1) (layer F.Cu) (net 4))
 (segment (start 188.849 83.693) (end 181.5846 83.693) (width 1) (layer F.Cu) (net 4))
 (segment (start 189.865 82.677) (end 188.849 83.693) (width 1) (layer F.Cu) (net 4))
 (segment (start 189.865 75.057) (end 189.865 82.677) (width 1) (layer F.Cu) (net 4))
 (segment (start 190.5 74.422) (end 189.865 75.057) (width 1) (layer F.Cu) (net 4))
 (segment (start 181.5846 83.693) (end 180.5432 82.6516) (width 1) (layer F.Cu) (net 4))
 (segment (start 191.897 57.15) (end 191.897 58.547) (width 1) (layer B.Cu) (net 4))
 (segment (start 192.278 73.152) (end 190.5 73.152) (width 1) (layer B.Cu) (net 4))
 (segment (start 192.278 58.928) (end 192.278 73.152) (width 1) (layer B.Cu) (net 4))
 (segment (start 191.897 58.547) (end 192.278 58.928) (width 1) (layer B.Cu) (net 4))
 (segment (start 187.132 73.914) (end 189.738 73.914) (width 1) (layer B.Cu) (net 4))
 (segment (start 189.738 73.914) (end 190.5 73.152) (width 1) (layer B.Cu) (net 4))
 (segment (start 187.132 71.882) (end 190.5 71.882) (width 1) (layer B.Cu) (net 8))
 (segment (start 187.0075 59.1185) (end 187.0075 57.9755) (width 1) (layer F.Cu) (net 6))
 (segment (start 177.626 56.896) (end 175.34 59.182) (width 1) (layer F.Cu) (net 6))
 (segment (start 185.928 56.896) (end 177.626 56.896) (width 1) (layer F.Cu) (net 6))
 (segment (start 187.0075 57.9755) (end 185.928 56.896) (width 1) (layer F.Cu) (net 6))
 (segment (start 180.34 59.182) (end 180.34 66.548) (width 2) (layer F.Cu) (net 7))
 (segment (start 182.2936 68.5016) (end 186.5932 68.5016) (width 2) (layer F.Cu) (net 7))
 (segment (start 180.34 66.548) (end 182.2936 68.5016) (width 2) (layer F.Cu) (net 7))
 (segment (start 191.516 65.09) (end 191.516 63.076) (width 1) (layer F.Cu) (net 9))
 (segment (start 191.516 63.076) (end 191.6 62.992) (width 1) (layer F.Cu) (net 9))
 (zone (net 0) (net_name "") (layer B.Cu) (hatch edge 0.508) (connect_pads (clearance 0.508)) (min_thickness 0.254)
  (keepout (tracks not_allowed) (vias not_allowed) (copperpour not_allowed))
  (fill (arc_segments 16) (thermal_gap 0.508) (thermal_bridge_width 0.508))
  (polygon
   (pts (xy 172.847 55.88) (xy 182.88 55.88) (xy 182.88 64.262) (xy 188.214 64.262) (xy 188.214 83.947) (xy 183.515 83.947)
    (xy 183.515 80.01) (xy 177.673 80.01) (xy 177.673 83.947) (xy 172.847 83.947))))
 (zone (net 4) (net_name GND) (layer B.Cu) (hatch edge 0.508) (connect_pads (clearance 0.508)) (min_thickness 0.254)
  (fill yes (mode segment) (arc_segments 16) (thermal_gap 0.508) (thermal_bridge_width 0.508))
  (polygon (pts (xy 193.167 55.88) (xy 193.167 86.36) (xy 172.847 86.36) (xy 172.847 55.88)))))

